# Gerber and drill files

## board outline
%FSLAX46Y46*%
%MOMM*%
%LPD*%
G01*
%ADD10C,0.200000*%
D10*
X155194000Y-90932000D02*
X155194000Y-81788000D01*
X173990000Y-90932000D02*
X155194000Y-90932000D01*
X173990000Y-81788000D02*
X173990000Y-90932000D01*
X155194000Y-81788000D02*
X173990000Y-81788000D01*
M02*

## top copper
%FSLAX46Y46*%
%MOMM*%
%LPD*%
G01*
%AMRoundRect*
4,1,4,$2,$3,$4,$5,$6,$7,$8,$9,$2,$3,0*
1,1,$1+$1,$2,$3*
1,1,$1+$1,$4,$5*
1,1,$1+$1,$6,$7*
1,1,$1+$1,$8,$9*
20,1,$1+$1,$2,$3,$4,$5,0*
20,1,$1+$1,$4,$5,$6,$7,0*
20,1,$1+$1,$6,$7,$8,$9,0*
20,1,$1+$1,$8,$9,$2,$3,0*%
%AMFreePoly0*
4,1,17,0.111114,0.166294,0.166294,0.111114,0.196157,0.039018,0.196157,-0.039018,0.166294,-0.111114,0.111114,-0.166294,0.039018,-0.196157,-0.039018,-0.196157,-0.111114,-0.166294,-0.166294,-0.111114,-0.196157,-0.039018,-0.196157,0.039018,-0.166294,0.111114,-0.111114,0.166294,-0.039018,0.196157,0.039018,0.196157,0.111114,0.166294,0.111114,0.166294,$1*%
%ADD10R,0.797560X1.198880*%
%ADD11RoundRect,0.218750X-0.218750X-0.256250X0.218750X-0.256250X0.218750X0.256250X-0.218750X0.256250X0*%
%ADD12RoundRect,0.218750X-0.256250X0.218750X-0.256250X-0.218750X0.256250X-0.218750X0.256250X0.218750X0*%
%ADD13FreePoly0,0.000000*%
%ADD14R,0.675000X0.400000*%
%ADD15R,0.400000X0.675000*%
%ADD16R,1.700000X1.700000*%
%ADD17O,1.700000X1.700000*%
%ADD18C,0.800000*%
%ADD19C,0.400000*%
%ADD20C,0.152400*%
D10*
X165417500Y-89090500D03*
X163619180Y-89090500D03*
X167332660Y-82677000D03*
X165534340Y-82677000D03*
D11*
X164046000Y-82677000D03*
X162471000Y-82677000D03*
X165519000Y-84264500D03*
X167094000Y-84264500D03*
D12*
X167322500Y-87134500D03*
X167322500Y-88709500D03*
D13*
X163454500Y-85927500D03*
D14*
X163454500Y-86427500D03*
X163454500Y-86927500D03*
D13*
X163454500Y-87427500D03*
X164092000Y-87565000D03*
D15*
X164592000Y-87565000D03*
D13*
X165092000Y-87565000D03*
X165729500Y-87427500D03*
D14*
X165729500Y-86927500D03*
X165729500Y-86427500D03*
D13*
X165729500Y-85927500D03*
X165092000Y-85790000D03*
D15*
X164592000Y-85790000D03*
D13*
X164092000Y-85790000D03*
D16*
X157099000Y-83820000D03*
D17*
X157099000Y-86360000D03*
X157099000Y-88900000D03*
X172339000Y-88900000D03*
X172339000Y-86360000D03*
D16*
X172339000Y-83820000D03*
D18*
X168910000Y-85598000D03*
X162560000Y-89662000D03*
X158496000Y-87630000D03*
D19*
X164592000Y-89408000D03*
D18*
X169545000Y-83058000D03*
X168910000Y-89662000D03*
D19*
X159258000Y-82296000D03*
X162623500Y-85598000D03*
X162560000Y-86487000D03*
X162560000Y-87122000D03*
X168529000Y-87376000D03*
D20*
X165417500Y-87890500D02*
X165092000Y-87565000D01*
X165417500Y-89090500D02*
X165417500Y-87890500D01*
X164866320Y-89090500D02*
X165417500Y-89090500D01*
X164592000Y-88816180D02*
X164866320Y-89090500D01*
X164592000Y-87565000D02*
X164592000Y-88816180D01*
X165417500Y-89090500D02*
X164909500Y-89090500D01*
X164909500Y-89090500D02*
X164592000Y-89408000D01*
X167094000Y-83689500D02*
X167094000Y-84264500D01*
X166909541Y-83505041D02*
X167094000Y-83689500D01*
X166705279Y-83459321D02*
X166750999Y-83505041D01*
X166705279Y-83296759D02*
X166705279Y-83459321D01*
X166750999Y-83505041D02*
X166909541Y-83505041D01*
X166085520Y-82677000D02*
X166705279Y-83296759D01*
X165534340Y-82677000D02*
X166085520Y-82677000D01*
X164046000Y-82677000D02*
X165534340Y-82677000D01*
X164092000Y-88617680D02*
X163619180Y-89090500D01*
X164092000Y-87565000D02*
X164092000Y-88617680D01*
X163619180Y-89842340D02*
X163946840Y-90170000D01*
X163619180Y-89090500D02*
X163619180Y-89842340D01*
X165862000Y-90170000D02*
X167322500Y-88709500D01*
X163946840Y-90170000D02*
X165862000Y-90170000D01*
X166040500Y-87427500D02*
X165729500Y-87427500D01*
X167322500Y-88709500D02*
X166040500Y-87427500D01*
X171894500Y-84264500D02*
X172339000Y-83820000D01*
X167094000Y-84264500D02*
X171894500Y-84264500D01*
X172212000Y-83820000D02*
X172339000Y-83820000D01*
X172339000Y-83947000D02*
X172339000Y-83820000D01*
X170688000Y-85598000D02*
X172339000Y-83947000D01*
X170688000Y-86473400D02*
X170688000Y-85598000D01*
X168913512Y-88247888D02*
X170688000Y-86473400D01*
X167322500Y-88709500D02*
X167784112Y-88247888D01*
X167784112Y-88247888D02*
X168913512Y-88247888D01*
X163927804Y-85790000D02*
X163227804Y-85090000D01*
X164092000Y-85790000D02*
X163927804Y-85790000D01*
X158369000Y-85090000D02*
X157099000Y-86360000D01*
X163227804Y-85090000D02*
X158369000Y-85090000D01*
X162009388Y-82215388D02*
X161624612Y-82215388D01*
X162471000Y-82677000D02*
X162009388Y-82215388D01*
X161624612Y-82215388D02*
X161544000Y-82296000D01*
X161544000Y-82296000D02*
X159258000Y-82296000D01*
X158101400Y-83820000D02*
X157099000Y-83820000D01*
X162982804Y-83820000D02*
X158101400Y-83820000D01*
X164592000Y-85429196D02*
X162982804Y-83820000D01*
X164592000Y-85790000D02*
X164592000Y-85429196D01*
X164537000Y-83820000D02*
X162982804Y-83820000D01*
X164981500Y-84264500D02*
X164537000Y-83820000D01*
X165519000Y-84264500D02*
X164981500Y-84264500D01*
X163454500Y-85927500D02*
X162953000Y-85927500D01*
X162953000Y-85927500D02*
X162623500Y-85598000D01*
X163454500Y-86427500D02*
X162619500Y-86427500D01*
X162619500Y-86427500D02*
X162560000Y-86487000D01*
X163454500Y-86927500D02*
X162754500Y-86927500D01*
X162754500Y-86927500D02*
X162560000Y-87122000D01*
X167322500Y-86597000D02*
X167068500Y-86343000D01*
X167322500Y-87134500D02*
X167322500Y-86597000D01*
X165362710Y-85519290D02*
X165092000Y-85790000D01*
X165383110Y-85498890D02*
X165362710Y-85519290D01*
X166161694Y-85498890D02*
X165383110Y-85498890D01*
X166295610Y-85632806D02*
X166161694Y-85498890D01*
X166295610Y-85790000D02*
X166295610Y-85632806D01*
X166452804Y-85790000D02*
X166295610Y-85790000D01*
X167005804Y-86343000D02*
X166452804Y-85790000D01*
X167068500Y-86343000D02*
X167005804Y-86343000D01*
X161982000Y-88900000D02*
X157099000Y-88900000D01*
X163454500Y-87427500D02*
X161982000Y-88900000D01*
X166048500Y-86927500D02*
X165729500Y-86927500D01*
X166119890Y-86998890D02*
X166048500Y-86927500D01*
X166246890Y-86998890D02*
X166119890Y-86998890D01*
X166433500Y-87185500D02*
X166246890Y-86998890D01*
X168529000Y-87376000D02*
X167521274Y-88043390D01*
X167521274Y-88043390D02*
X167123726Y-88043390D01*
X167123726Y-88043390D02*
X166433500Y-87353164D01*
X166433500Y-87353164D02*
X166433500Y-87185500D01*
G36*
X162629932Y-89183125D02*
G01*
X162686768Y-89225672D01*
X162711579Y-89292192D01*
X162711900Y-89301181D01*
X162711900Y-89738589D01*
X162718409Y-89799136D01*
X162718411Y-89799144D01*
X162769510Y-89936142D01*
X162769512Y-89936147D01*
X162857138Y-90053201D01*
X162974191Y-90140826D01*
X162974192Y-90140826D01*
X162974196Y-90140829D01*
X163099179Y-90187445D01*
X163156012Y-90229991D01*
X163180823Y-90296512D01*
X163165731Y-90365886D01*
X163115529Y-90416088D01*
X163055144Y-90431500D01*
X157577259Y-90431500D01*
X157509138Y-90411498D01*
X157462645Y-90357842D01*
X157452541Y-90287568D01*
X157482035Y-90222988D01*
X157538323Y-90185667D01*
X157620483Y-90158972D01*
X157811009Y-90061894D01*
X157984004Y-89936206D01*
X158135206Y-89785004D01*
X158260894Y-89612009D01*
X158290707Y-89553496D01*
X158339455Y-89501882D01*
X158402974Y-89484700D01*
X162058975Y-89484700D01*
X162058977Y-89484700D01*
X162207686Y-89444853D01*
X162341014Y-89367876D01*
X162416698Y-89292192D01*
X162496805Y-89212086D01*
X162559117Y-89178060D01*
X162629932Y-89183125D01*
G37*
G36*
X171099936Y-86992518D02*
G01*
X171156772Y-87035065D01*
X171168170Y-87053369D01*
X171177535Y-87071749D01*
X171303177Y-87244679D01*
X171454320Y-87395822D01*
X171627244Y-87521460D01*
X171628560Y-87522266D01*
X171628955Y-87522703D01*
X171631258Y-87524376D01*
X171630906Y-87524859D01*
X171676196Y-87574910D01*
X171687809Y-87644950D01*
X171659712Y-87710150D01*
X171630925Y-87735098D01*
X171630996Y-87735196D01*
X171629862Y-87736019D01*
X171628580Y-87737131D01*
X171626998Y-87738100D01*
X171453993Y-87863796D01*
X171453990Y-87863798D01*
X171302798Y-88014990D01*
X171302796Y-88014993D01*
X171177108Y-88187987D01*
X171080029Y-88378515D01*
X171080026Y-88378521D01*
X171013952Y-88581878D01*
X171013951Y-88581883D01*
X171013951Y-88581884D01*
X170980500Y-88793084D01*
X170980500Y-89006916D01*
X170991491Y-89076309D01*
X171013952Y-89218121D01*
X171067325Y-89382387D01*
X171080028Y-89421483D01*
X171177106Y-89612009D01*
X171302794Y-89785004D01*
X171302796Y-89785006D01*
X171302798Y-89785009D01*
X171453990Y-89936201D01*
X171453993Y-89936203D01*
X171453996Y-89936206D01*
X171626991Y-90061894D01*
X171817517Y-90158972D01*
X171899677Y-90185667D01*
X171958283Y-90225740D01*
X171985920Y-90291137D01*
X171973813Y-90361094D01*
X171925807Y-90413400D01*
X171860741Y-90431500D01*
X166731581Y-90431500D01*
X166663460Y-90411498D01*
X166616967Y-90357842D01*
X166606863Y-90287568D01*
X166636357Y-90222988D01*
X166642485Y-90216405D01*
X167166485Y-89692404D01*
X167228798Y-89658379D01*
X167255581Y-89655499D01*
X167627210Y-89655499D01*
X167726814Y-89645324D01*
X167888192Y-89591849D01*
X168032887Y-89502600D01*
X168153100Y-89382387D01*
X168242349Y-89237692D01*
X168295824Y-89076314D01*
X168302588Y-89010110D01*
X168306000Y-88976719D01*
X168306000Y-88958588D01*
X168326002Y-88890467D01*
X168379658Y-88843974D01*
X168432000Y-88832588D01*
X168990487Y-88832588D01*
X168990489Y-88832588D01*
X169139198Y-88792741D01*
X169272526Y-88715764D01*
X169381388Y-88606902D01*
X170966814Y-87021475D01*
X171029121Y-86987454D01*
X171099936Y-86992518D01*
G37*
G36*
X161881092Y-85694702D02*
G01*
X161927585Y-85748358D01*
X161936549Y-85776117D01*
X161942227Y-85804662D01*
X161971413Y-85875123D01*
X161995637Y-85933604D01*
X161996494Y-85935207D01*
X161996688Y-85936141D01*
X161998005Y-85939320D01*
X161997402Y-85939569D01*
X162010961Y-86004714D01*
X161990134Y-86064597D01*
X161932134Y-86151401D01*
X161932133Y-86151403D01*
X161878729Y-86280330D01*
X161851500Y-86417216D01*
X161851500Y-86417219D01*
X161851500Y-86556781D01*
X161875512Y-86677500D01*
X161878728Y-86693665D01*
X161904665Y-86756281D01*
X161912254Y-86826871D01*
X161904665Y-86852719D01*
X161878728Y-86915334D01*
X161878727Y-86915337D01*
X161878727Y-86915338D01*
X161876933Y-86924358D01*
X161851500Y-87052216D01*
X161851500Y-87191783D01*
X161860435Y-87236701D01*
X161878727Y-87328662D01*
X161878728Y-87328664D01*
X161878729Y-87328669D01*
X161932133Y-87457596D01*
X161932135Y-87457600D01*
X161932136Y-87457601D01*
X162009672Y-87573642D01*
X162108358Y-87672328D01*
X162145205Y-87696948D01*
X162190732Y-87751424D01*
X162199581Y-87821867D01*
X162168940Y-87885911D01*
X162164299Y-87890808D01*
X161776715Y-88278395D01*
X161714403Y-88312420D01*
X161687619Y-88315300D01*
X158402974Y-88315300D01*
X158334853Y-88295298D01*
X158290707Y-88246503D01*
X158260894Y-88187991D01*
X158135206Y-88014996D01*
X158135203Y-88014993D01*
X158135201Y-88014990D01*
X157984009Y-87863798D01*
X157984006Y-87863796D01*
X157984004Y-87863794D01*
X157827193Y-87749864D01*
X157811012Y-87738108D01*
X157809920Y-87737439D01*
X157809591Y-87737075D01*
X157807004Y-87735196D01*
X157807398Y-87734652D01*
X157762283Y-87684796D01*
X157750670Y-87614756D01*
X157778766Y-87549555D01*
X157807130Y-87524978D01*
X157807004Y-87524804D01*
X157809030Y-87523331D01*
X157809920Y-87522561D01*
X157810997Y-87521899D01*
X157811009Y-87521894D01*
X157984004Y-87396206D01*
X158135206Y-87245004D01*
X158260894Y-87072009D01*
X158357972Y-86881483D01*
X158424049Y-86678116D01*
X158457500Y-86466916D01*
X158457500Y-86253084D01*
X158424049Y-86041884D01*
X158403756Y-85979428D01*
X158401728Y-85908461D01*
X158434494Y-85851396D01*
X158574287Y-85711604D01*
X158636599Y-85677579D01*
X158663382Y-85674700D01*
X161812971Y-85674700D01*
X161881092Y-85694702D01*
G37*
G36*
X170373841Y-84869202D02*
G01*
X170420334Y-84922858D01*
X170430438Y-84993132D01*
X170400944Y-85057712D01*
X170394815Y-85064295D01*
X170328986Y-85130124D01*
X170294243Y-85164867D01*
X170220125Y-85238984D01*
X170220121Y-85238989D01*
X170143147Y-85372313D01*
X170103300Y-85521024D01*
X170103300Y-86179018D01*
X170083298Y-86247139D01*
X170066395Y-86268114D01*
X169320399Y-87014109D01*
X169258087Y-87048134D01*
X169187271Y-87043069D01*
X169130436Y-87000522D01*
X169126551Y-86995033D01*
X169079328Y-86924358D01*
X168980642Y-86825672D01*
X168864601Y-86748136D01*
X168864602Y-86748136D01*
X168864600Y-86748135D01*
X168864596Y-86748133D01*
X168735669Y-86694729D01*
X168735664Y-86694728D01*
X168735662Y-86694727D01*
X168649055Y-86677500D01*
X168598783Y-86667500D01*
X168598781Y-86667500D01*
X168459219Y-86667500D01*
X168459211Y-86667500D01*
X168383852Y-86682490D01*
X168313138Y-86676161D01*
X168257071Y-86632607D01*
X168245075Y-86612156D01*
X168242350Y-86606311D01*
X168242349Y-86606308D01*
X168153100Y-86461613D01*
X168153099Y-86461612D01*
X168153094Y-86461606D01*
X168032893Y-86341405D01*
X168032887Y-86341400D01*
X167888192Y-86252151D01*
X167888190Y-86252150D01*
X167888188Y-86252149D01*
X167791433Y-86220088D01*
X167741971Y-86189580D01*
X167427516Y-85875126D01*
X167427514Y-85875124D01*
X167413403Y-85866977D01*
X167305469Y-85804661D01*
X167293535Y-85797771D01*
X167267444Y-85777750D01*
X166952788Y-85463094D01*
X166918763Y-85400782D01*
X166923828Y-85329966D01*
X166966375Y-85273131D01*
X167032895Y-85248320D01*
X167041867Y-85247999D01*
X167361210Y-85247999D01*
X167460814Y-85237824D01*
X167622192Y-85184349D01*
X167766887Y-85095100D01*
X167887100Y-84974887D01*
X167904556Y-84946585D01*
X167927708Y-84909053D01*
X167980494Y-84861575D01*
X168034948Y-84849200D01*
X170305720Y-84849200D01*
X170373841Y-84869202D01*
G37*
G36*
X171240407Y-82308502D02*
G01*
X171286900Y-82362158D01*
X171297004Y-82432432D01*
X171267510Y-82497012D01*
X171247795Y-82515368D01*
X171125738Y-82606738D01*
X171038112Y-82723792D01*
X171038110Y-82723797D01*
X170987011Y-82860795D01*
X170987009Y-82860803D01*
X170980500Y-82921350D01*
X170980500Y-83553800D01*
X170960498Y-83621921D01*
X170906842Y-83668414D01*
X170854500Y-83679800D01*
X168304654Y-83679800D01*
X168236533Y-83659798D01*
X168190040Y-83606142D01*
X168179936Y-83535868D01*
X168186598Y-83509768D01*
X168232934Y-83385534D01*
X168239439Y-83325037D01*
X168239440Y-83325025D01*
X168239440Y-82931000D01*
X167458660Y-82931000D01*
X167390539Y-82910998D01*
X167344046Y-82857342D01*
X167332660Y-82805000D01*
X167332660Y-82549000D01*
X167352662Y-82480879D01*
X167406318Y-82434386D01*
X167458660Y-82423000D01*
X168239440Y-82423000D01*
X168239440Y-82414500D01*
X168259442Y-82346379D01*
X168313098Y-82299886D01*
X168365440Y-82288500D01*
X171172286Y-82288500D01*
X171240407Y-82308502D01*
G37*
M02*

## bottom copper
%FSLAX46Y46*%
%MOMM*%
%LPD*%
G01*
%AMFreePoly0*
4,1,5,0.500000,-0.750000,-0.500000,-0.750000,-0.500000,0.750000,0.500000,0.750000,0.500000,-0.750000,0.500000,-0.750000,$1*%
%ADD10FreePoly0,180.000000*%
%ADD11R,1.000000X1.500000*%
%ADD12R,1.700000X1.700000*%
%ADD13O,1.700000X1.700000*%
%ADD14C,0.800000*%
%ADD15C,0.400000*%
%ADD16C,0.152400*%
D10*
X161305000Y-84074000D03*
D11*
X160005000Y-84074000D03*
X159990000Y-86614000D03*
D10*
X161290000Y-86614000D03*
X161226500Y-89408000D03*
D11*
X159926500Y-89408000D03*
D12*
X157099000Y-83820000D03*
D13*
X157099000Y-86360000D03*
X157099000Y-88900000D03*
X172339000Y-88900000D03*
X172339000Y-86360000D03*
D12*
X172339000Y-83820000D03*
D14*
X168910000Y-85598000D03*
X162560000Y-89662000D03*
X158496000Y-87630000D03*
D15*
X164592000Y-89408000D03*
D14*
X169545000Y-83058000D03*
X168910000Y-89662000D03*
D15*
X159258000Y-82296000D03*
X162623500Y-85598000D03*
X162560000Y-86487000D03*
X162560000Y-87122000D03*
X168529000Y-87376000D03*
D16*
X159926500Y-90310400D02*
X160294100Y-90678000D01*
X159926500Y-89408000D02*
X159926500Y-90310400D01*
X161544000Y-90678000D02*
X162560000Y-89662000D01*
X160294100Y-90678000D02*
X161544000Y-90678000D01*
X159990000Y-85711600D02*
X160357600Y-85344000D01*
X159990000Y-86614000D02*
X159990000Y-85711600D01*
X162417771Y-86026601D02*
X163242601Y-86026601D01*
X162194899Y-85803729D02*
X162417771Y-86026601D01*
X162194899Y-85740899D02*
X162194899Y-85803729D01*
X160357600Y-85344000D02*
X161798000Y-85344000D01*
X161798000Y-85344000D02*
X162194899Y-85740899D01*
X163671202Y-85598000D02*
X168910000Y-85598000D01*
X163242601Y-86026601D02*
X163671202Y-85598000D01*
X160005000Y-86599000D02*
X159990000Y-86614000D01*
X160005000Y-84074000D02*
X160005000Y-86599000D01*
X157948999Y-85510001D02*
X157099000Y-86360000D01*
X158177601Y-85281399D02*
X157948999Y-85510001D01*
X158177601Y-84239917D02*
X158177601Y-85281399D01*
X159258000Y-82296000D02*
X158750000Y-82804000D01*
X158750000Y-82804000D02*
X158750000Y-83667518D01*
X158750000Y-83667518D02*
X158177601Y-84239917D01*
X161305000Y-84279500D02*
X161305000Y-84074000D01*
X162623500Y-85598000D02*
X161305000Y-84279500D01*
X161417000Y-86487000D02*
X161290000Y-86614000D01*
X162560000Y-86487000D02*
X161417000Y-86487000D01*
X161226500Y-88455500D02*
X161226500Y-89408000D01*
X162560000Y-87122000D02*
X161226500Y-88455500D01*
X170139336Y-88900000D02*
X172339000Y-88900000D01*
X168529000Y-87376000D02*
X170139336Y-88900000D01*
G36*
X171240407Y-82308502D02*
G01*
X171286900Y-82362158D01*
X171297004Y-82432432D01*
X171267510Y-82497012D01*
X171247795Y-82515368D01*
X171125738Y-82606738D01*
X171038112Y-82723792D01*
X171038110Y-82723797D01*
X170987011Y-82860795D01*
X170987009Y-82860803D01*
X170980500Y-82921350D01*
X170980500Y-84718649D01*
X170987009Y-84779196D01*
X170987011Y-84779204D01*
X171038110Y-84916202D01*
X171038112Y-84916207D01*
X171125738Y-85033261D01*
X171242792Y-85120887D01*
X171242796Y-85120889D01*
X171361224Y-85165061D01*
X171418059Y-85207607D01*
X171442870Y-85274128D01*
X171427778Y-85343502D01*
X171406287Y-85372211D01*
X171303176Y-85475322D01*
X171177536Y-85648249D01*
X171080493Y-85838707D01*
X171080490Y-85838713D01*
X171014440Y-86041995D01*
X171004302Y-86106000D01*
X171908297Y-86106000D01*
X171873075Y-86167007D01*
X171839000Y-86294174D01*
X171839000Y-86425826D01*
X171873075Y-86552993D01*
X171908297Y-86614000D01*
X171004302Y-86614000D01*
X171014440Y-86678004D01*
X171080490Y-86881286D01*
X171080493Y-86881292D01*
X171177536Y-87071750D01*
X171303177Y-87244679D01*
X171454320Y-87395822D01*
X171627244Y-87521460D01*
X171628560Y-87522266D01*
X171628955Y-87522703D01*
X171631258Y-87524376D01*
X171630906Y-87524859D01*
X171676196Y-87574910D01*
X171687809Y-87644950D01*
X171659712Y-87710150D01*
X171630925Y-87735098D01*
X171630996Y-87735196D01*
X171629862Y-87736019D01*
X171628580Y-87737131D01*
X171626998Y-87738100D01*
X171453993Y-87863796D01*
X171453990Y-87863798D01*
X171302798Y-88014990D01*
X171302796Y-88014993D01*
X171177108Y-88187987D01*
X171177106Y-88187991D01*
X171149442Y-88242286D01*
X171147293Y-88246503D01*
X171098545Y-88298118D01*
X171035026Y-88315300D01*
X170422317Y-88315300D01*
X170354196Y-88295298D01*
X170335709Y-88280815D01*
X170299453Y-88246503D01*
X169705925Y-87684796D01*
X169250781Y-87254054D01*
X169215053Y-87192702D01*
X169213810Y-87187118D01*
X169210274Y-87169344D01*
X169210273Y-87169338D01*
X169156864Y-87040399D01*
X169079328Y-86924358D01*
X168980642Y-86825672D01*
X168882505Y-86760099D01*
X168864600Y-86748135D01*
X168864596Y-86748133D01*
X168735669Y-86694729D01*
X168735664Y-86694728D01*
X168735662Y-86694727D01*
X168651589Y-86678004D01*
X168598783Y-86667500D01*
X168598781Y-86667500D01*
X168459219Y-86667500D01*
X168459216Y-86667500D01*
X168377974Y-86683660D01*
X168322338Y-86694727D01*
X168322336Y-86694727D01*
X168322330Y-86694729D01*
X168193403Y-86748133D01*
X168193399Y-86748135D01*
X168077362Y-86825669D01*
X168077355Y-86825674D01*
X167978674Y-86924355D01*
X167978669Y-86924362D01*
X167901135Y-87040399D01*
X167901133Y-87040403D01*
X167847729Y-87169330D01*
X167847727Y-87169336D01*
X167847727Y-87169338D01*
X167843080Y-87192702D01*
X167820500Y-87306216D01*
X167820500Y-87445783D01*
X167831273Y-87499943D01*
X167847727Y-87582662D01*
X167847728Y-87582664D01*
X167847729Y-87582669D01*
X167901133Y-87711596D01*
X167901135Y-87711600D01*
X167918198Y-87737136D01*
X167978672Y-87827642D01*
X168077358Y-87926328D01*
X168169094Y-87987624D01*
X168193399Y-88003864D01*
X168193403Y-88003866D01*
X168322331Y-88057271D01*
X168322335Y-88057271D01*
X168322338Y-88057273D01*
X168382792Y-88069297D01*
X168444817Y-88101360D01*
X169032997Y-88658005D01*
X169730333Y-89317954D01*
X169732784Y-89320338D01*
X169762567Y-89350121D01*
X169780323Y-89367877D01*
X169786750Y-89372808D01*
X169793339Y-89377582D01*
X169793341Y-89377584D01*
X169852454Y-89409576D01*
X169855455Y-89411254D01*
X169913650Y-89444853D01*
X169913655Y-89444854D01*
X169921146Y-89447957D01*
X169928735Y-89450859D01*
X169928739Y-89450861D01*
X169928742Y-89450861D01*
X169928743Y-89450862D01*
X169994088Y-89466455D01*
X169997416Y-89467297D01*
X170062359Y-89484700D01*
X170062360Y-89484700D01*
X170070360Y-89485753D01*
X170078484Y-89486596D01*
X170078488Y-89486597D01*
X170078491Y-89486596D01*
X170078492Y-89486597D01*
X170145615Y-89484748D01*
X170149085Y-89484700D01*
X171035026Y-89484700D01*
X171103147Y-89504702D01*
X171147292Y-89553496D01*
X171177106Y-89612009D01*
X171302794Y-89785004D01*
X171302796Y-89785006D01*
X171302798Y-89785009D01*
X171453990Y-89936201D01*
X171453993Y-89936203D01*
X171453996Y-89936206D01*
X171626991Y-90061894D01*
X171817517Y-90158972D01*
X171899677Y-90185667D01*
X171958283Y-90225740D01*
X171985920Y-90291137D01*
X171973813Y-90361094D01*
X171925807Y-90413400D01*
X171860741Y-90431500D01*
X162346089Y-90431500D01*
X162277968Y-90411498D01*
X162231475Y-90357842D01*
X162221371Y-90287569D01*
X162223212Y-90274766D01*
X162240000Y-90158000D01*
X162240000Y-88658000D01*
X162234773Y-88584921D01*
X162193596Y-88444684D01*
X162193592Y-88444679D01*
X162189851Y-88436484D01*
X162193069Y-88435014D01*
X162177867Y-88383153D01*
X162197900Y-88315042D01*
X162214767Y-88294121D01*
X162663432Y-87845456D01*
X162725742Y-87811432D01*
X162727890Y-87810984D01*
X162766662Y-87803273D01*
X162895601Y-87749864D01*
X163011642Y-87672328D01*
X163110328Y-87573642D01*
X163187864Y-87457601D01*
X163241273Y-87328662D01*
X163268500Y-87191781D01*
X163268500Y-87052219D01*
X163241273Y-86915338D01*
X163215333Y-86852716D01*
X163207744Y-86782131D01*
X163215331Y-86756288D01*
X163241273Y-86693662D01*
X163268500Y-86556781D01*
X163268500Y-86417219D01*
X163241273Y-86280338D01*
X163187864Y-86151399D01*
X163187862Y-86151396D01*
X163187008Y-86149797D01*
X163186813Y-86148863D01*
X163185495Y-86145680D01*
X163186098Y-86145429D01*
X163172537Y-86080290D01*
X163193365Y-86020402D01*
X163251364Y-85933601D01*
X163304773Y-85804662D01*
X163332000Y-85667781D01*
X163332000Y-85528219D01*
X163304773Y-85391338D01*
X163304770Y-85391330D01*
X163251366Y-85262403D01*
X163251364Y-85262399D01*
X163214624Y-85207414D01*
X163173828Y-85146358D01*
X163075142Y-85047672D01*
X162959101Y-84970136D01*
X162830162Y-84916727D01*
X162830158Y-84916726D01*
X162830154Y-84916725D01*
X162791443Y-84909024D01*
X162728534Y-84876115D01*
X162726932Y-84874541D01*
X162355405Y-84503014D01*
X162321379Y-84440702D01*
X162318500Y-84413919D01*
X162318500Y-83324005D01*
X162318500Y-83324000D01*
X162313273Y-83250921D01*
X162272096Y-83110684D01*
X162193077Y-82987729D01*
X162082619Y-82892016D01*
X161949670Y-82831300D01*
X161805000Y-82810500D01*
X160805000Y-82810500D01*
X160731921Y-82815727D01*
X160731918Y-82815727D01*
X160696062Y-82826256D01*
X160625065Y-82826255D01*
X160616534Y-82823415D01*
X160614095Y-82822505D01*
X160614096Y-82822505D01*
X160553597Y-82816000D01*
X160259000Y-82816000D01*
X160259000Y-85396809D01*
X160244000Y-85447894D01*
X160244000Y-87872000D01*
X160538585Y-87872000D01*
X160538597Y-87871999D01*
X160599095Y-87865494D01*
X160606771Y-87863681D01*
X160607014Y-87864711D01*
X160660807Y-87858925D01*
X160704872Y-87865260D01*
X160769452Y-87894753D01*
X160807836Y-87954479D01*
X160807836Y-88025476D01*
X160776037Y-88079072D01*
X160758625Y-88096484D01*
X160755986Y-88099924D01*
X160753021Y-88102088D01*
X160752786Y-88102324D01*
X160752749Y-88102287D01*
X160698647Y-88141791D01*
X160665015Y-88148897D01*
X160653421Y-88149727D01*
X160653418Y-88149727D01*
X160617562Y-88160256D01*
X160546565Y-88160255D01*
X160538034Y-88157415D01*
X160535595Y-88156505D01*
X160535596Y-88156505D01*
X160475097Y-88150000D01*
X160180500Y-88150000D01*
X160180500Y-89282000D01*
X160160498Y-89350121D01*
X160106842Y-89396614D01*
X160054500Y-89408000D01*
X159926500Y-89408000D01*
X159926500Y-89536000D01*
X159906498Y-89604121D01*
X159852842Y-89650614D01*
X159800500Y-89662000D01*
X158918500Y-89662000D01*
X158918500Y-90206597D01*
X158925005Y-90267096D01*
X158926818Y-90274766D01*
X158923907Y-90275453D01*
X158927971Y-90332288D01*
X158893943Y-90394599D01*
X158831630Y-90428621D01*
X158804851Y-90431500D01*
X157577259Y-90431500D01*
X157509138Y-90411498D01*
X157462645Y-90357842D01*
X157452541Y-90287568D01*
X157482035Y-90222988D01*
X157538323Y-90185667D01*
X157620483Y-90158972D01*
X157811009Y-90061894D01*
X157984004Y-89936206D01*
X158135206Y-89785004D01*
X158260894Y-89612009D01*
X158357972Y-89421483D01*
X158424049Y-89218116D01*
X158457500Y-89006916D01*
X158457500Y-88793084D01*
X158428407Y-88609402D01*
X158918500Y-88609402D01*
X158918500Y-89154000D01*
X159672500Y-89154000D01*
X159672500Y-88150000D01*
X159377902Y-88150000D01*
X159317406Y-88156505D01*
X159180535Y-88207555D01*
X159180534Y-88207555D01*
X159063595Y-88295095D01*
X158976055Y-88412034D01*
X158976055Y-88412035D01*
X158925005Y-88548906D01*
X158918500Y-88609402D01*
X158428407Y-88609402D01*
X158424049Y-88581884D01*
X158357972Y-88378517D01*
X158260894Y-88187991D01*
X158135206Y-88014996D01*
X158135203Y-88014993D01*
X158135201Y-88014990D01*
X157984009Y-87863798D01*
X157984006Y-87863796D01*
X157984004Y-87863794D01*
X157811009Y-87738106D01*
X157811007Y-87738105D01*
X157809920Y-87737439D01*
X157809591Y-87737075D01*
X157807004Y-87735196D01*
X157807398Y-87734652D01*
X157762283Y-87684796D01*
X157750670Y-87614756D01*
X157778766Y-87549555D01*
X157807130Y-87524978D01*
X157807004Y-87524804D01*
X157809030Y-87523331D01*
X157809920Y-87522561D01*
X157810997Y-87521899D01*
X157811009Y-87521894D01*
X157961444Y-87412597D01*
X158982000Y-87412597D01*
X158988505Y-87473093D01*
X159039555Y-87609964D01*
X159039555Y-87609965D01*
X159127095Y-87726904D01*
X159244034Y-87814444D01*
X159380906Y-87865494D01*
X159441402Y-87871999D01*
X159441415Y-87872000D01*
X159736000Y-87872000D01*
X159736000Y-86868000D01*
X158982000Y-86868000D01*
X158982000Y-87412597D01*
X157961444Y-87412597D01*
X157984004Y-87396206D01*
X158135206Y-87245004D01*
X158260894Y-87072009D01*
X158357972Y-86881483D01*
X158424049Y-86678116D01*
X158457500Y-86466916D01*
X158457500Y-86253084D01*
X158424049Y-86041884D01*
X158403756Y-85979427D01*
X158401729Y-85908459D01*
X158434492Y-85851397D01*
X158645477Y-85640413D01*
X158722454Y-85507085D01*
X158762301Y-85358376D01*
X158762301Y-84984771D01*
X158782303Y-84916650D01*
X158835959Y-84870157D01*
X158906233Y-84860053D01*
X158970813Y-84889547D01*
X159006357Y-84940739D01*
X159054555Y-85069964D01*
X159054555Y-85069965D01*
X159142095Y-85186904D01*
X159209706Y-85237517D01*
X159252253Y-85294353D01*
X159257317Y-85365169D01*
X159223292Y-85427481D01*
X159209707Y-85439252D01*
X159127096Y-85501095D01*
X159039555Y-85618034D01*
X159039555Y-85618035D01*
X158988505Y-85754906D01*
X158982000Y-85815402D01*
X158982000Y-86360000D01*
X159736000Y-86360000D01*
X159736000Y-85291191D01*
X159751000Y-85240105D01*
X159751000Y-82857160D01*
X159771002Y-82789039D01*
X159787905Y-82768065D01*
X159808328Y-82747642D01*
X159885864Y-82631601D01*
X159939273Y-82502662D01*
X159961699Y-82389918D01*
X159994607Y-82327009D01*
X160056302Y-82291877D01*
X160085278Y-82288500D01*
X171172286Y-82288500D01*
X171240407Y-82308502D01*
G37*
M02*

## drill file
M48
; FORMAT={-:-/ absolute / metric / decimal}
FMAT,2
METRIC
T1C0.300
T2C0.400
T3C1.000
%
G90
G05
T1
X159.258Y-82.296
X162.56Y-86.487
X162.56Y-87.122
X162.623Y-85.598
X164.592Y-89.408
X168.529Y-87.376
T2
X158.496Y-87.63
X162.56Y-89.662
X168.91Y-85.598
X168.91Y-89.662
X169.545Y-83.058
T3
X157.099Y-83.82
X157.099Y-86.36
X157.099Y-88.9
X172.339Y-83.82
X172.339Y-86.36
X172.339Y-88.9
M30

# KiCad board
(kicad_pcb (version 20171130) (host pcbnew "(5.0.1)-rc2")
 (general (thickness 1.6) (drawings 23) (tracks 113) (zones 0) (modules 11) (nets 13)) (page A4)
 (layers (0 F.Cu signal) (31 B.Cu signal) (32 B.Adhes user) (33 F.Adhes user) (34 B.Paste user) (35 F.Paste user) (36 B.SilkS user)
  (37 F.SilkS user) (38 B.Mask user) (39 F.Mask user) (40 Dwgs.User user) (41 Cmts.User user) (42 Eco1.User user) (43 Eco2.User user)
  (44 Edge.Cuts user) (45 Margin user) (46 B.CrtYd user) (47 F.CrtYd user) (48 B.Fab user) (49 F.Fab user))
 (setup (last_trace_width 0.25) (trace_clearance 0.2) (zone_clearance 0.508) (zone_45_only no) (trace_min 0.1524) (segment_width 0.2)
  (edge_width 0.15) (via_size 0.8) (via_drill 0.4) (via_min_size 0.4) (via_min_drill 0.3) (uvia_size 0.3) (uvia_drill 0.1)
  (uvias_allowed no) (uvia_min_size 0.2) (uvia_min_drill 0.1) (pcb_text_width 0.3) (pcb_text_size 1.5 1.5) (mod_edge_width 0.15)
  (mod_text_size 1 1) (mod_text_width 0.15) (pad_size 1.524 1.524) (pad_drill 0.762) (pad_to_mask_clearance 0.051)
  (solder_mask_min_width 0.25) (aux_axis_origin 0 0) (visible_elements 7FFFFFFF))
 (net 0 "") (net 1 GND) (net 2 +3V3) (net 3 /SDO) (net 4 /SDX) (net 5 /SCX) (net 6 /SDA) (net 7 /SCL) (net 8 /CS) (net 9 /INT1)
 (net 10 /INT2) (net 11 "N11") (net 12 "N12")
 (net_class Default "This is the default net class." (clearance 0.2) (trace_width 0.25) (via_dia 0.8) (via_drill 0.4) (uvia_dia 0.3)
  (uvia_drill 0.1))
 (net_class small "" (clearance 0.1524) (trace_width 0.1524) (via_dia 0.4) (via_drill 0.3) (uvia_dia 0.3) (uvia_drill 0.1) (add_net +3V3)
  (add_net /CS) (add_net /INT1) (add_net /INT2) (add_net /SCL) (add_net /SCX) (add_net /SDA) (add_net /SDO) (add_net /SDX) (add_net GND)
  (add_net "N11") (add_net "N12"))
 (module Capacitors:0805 (layer F.Cu) (at 164.51834 89.0905 180)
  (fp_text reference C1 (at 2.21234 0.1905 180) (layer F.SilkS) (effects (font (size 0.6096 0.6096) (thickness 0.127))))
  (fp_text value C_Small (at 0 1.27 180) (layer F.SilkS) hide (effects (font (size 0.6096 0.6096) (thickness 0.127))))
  (pad 1 smd rect (at -0.89916 0 180) (size 0.79756 1.19888) (layers F.Cu F.Paste F.Mask) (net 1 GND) (solder_mask_margin 0.1016))
  (pad 2 smd rect (at 0.89916 0 180) (size 0.79756 1.19888) (layers F.Cu F.Paste F.Mask) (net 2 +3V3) (solder_mask_margin 0.1016)))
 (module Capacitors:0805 (layer F.Cu) (at 166.4335 82.677)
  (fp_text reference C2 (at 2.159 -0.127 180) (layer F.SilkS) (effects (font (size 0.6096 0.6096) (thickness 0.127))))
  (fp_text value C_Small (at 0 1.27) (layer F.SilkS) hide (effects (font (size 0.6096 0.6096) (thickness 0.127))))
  (pad 2 smd rect (at 0.89916 0) (size 0.79756 1.19888) (layers F.Cu F.Paste F.Mask) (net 1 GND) (solder_mask_margin 0.1016))
  (pad 1 smd rect (at -0.89916 0) (size 0.79756 1.19888) (layers F.Cu F.Paste F.Mask) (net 2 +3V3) (solder_mask_margin 0.1016)))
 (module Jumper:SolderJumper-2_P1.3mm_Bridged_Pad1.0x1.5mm (layer B.Cu) (at 160.655 84.074 180)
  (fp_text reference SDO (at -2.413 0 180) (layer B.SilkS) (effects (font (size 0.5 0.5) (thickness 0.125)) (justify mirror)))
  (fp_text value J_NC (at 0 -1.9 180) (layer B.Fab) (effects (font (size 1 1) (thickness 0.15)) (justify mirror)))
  (pad 1 smd custom (at -0.65 0 180) (size 1 1.5) (layers B.Cu B.Mask) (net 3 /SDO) (options (clearance outline) (anchor rect)) (primitives))
  (pad 2 smd rect (at 0.65 0 180) (size 1 1.5) (layers B.Cu B.Mask) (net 1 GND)))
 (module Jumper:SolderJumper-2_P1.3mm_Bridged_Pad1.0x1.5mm (layer B.Cu) (at 160.64 86.614 180)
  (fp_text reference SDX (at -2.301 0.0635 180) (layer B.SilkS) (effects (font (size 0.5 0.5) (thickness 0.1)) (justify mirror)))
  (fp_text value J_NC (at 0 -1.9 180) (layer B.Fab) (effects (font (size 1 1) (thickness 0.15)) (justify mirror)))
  (pad 2 smd rect (at 0.65 0 180) (size 1 1.5) (layers B.Cu B.Mask) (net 1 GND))
  (pad 1 smd custom (at -0.65 0 180) (size 1 1.5) (layers B.Cu B.Mask) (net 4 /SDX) (options (clearance outline) (anchor rect)) (primitives)))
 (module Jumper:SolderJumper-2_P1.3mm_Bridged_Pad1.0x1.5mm (layer B.Cu) (at 160.5765 89.408 180)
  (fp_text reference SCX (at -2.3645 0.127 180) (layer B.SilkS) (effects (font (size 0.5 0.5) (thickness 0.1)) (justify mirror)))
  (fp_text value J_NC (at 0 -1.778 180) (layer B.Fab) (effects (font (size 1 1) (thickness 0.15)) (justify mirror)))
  (pad 1 smd custom (at -0.65 0 180) (size 1 1.5) (layers B.Cu B.Mask) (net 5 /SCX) (options (clearance outline) (anchor rect)) (primitives))
  (pad 2 smd rect (at 0.65 0 180) (size 1 1.5) (layers B.Cu B.Mask) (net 1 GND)))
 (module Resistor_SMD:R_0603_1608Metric (layer F.Cu) (at 163.2585 82.677)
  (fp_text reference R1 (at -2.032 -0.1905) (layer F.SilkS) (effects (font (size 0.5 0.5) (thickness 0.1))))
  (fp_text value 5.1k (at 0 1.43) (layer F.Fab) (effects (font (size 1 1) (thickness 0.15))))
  (pad 2 smd roundrect (at 0.7875 0) (size 0.875 0.95) (layers F.Cu F.Paste F.Mask) (roundrect_rratio 0.25) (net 2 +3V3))
  (pad 1 smd roundrect (at -0.7875 0) (size 0.875 0.95) (layers F.Cu F.Paste F.Mask) (roundrect_rratio 0.25) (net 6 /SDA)))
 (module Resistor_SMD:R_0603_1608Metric (layer F.Cu) (at 166.3065 84.2645)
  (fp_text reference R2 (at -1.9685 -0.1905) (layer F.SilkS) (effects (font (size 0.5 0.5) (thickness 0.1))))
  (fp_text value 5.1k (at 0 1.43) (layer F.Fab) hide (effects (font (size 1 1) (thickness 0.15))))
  (pad 1 smd roundrect (at -0.7875 0) (size 0.875 0.95) (layers F.Cu F.Paste F.Mask) (roundrect_rratio 0.25) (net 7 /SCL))
  (pad 2 smd roundrect (at 0.7875 0) (size 0.875 0.95) (layers F.Cu F.Paste F.Mask) (roundrect_rratio 0.25) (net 2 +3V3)))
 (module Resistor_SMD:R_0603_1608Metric (layer F.Cu) (at 167.3225 87.922 270)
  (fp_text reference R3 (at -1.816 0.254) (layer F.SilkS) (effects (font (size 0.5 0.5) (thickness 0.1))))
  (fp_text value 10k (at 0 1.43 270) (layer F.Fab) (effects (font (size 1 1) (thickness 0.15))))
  (pad 1 smd roundrect (at -0.7875 0 270) (size 0.875 0.95) (layers F.Cu F.Paste F.Mask) (roundrect_rratio 0.25) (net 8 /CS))
  (pad 2 smd roundrect (at 0.7875 0 270) (size 0.875 0.95) (layers F.Cu F.Paste F.Mask) (roundrect_rratio 0.25) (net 2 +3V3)))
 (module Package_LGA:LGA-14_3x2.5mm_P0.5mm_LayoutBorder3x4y (layer F.Cu) (at 164.592 86.6775)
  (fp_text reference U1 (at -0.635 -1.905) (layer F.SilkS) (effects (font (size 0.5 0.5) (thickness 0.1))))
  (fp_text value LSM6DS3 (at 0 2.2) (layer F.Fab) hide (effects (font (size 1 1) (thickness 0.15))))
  (pad 1 smd custom (at -1.1375 -0.75) (size 0.4 0.4) (layers F.Cu F.Paste F.Mask) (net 3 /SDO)
   (options (clearance outline) (anchor circle)) (primitives))
  (pad 2 smd rect (at -1.1375 -0.25) (size 0.675 0.4) (layers F.Cu F.Paste F.Mask) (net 4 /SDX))
  (pad 3 smd rect (at -1.1375 0.25) (size 0.675 0.4) (layers F.Cu F.Paste F.Mask) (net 5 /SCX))
  (pad 4 smd custom (at -1.1375 0.75) (size 0.4 0.4) (layers F.Cu F.Paste F.Mask) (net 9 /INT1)
   (options (clearance outline) (anchor circle)) (primitives))
  (pad 5 smd custom (at -0.5 0.8875) (size 0.4 0.4) (layers F.Cu F.Paste F.Mask) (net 2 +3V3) (options (clearance outline) (anchor circle))
   (primitives))
  (pad 6 smd rect (at 0 0.8875) (size 0.4 0.675) (layers F.Cu F.Paste F.Mask) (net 1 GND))
  (pad 7 smd custom (at 0.5 0.8875) (size 0.4 0.4) (layers F.Cu F.Paste F.Mask) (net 1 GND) (options (clearance outline) (anchor circle))
   (primitives))
  (pad 8 smd custom (at 1.1375 0.75) (size 0.4 0.4) (layers F.Cu F.Paste F.Mask) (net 2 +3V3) (options (clearance outline) (anchor circle))
   (primitives))
  (pad 9 smd rect (at 1.1375 0.25) (size 0.675 0.4) (layers F.Cu F.Paste F.Mask) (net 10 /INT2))
  (pad 10 smd rect (at 1.1375 -0.25) (size 0.675 0.4) (layers F.Cu F.Paste F.Mask) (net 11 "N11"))
  (pad 11 smd custom (at 1.1375 -0.75) (size 0.4 0.4) (layers F.Cu F.Paste F.Mask) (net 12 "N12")
   (options (clearance outline) (anchor circle)) (primitives))
  (pad 12 smd custom (at 0.5 -0.8875) (size 0.4 0.4) (layers F.Cu F.Paste F.Mask) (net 8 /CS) (options (clearance outline) (anchor circle))
   (primitives))
  (pad 13 smd rect (at 0 -0.8875) (size 0.4 0.675) (layers F.Cu F.Paste F.Mask) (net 7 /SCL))
  (pad 14 smd custom (at -0.5 -0.8875) (size 0.4 0.4) (layers F.Cu F.Paste F.Mask) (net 6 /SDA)
   (options (clearance outline) (anchor circle)) (primitives)))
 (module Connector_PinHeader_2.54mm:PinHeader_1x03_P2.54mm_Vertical (layer F.Cu) (at 157.099 83.82)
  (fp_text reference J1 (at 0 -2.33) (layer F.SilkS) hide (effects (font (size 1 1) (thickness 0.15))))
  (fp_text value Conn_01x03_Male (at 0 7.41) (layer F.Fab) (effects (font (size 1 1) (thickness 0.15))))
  (pad 1 thru_hole rect (at 0 0) (size 1.7 1.7) (drill 1) (layers *.Cu *.Mask) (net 7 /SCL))
  (pad 2 thru_hole oval (at 0 2.54) (size 1.7 1.7) (drill 1) (layers *.Cu *.Mask) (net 6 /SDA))
  (pad 3 thru_hole oval (at 0 5.08) (size 1.7 1.7) (drill 1) (layers *.Cu *.Mask) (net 9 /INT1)))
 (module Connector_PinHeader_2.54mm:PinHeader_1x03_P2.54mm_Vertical (layer F.Cu) (at 172.339 83.82)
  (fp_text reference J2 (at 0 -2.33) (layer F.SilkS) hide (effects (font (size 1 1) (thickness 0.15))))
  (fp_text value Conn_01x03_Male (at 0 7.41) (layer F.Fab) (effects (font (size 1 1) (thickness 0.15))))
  (pad 3 thru_hole oval (at 0 5.08) (size 1.7 1.7) (drill 1) (layers *.Cu *.Mask) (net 10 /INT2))
  (pad 2 thru_hole oval (at 0 2.54) (size 1.7 1.7) (drill 1) (layers *.Cu *.Mask) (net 1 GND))
  (pad 1 thru_hole rect (at 0 0) (size 1.7 1.7) (drill 1) (layers *.Cu *.Mask) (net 2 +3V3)))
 (gr_line (start 155.194 90.932) (end 155.194 81.788) (layer Edge.Cuts) (width 0.2))
 (gr_line (start 173.99 90.932) (end 155.194 90.932) (layer Edge.Cuts) (width 0.2))
 (gr_line (start 173.99 81.788) (end 173.99 90.932) (layer Edge.Cuts) (width 0.2))
 (gr_line (start 155.194 81.788) (end 173.99 81.788) (layer Edge.Cuts) (width 0.2))
 (via (at 168.91 85.598) (size 0.8) (drill 0.4) (layers F.Cu B.Cu) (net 1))
 (segment (start 165.4175 87.8905) (end 165.092 87.565) (width 0.1524) (layer F.Cu) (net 1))
 (segment (start 165.4175 89.0905) (end 165.4175 87.8905) (width 0.1524) (layer F.Cu) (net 1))
 (segment (start 164.86632 89.0905) (end 165.4175 89.0905) (width 0.1524) (layer F.Cu) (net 1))
 (segment (start 164.592 88.81618) (end 164.86632 89.0905) (width 0.1524) (layer F.Cu) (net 1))
 (segment (start 164.592 87.565) (end 164.592 88.81618) (width 0.1524) (layer F.Cu) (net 1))
 (via (at 162.56 89.662) (size 0.8) (drill 0.4) (layers F.Cu B.Cu) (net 1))
 (via (at 158.496 87.63) (size 0.8) (drill 0.4) (layers F.Cu B.Cu) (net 1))
 (segment (start 159.9265 90.3104) (end 160.2941 90.678) (width 0.1524) (layer B.Cu) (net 1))
 (segment (start 159.9265 89.408) (end 159.9265 90.3104) (width 0.1524) (layer B.Cu) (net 1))
 (segment (start 161.544 90.678) (end 162.56 89.662) (width 0.1524) (layer B.Cu) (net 1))
 (segment (start 160.2941 90.678) (end 161.544 90.678) (width 0.1524) (layer B.Cu) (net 1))
 (segment (start 159.99 85.7116) (end 160.3576 85.344) (width 0.1524) (layer B.Cu) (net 1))
 (segment (start 159.99 86.614) (end 159.99 85.7116) (width 0.1524) (layer B.Cu) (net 1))
 (segment (start 162.417771 86.026601) (end 163.242601 86.026601) (width 0.1524) (layer B.Cu) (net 1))
 (segment (start 162.194899 85.803729) (end 162.417771 86.026601) (width 0.1524) (layer B.Cu) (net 1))
 (segment (start 162.194899 85.740899) (end 162.194899 85.803729) (width 0.1524) (layer B.Cu) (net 1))
 (segment (start 160.3576 85.344) (end 161.798 85.344) (width 0.1524) (layer B.Cu) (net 1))
 (segment (start 161.798 85.344) (end 162.194899 85.740899) (width 0.1524) (layer B.Cu) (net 1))
 (segment (start 163.671202 85.598) (end 168.91 85.598) (width 0.1524) (layer B.Cu) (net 1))
 (segment (start 163.242601 86.026601) (end 163.671202 85.598) (width 0.1524) (layer B.Cu) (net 1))
 (segment (start 160.005 86.599) (end 159.99 86.614) (width 0.1524) (layer B.Cu) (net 1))
 (segment (start 160.005 84.074) (end 160.005 86.599) (width 0.1524) (layer B.Cu) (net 1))
 (via (at 164.592 89.408) (size 0.4) (drill 0.3) (layers F.Cu B.Cu) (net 1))
 (segment (start 165.4175 89.0905) (end 164.9095 89.0905) (width 0.1524) (layer F.Cu) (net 1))
 (segment (start 164.9095 89.0905) (end 164.592 89.408) (width 0.1524) (layer F.Cu) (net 1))
 (via (at 169.545 83.058) (size 0.8) (drill 0.4) (layers F.Cu B.Cu) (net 1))
 (via (at 168.91 89.662) (size 0.8) (drill 0.4) (layers F.Cu B.Cu) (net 1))
 (segment (start 167.094 83.6895) (end 167.094 84.2645) (width 0.1524) (layer F.Cu) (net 2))
 (segment (start 166.909541 83.505041) (end 167.094 83.6895) (width 0.1524) (layer F.Cu) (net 2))
 (segment (start 166.705279 83.459321) (end 166.750999 83.505041) (width 0.1524) (layer F.Cu) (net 2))
 (segment (start 166.705279 83.296759) (end 166.705279 83.459321) (width 0.1524) (layer F.Cu) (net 2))
 (segment (start 166.750999 83.505041) (end 166.909541 83.505041) (width 0.1524) (layer F.Cu) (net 2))
 (segment (start 166.08552 82.677) (end 166.705279 83.296759) (width 0.1524) (layer F.Cu) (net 2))
 (segment (start 165.53434 82.677) (end 166.08552 82.677) (width 0.1524) (layer F.Cu) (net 2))
 (segment (start 164.046 82.677) (end 165.53434 82.677) (width 0.1524) (layer F.Cu) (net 2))
 (segment (start 164.092 88.61768) (end 163.61918 89.0905) (width 0.1524) (layer F.Cu) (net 2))
 (segment (start 164.092 87.565) (end 164.092 88.61768) (width 0.1524) (layer F.Cu) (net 2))
 (segment (start 163.61918 89.84234) (end 163.94684 90.17) (width 0.1524) (layer F.Cu) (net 2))
 (segment (start 163.61918 89.0905) (end 163.61918 89.84234) (width 0.1524) (layer F.Cu) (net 2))
 (segment (start 165.862 90.17) (end 167.3225 88.7095) (width 0.1524) (layer F.Cu) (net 2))
 (segment (start 163.94684 90.17) (end 165.862 90.17) (width 0.1524) (layer F.Cu) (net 2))
 (segment (start 166.0405 87.4275) (end 165.7295 87.4275) (width 0.1524) (layer F.Cu) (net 2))
 (segment (start 167.3225 88.7095) (end 166.0405 87.4275) (width 0.1524) (layer F.Cu) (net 2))
 (segment (start 171.8945 84.2645) (end 172.339 83.82) (width 0.1524) (layer F.Cu) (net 2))
 (segment (start 167.094 84.2645) (end 171.8945 84.2645) (width 0.1524) (layer F.Cu) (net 2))
 (segment (start 172.212 83.82) (end 172.339 83.82) (width 0.1524) (layer F.Cu) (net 2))
 (segment (start 172.339 83.947) (end 172.339 83.82) (width 0.1524) (layer F.Cu) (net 2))
 (segment (start 170.688 85.598) (end 172.339 83.947) (width 0.1524) (layer F.Cu) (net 2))
 (segment (start 170.688 86.4734) (end 170.688 85.598) (width 0.1524) (layer F.Cu) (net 2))
 (segment (start 168.913512 88.247888) (end 170.688 86.4734) (width 0.1524) (layer F.Cu) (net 2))
 (segment (start 167.3225 88.7095) (end 167.784112 88.247888) (width 0.1524) (layer F.Cu) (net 2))
 (segment (start 167.784112 88.247888) (end 168.913512 88.247888) (width 0.1524) (layer F.Cu) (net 2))
 (segment (start 163.927804 85.79) (end 163.227804 85.09) (width 0.1524) (layer F.Cu) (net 6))
 (segment (start 164.092 85.79) (end 163.927804 85.79) (width 0.1524) (layer F.Cu) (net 6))
 (segment (start 158.369 85.09) (end 157.099 86.36) (width 0.1524) (layer F.Cu) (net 6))
 (segment (start 163.227804 85.09) (end 158.369 85.09) (width 0.1524) (layer F.Cu) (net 6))
 (segment (start 157.948999 85.510001) (end 157.099 86.36) (width 0.1524) (layer B.Cu) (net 6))
 (segment (start 158.177601 85.281399) (end 157.948999 85.510001) (width 0.1524) (layer B.Cu) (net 6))
 (segment (start 158.177601 84.239917) (end 158.177601 85.281399) (width 0.1524) (layer B.Cu) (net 6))
 (segment (start 162.009388 82.215388) (end 161.624612 82.215388) (width 0.1524) (layer F.Cu) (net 6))
 (segment (start 162.471 82.677) (end 162.009388 82.215388) (width 0.1524) (layer F.Cu) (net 6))
 (segment (start 161.624612 82.215388) (end 161.544 82.296) (width 0.1524) (layer F.Cu) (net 6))
 (via (at 159.258 82.296) (size 0.4) (drill 0.3) (layers F.Cu B.Cu) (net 6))
 (segment (start 161.544 82.296) (end 159.258 82.296) (width 0.1524) (layer F.Cu) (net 6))
 (segment (start 159.258 82.296) (end 158.75 82.804) (width 0.1524) (layer B.Cu) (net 6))
 (segment (start 158.75 82.804) (end 158.75 83.667518) (width 0.1524) (layer B.Cu) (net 6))
 (segment (start 158.75 83.667518) (end 158.177601 84.239917) (width 0.1524) (layer B.Cu) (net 6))
 (segment (start 158.1014 83.82) (end 157.099 83.82) (width 0.1524) (layer F.Cu) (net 7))
 (segment (start 162.982804 83.82) (end 158.1014 83.82) (width 0.1524) (layer F.Cu) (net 7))
 (segment (start 164.592 85.429196) (end 162.982804 83.82) (width 0.1524) (layer F.Cu) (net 7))
 (segment (start 164.592 85.79) (end 164.592 85.429196) (width 0.1524) (layer F.Cu) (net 7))
 (segment (start 164.537 83.82) (end 162.982804 83.82) (width 0.1524) (layer F.Cu) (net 7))
 (segment (start 164.9815 84.2645) (end 164.537 83.82) (width 0.1524) (layer F.Cu) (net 7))
 (segment (start 165.519 84.2645) (end 164.9815 84.2645) (width 0.1524) (layer F.Cu) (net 7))
 (via (at 162.6235 85.598) (size 0.4) (drill 0.3) (layers F.Cu B.Cu) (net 3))
 (segment (start 163.4545 85.9275) (end 162.953 85.9275) (width 0.1524) (layer F.Cu) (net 3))
 (segment (start 162.953 85.9275) (end 162.6235 85.598) (width 0.1524) (layer F.Cu) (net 3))
 (segment (start 161.305 84.2795) (end 161.305 84.074) (width 0.1524) (layer B.Cu) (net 3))
 (segment (start 162.6235 85.598) (end 161.305 84.2795) (width 0.1524) (layer B.Cu) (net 3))
 (via (at 162.56 86.487) (size 0.4) (drill 0.3) (layers F.Cu B.Cu) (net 4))
 (segment (start 163.4545 86.4275) (end 162.6195 86.4275) (width 0.1524) (layer F.Cu) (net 4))
 (segment (start 162.6195 86.4275) (end 162.56 86.487) (width 0.1524) (layer F.Cu) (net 4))
 (segment (start 161.417 86.487) (end 161.29 86.614) (width 0.1524) (layer B.Cu) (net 4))
 (segment (start 162.56 86.487) (end 161.417 86.487) (width 0.1524) (layer B.Cu) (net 4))
 (via (at 162.56 87.122) (size 0.4) (drill 0.3) (layers F.Cu B.Cu) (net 5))
 (segment (start 163.4545 86.9275) (end 162.7545 86.9275) (width 0.1524) (layer F.Cu) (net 5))
 (segment (start 162.7545 86.9275) (end 162.56 87.122) (width 0.1524) (layer F.Cu) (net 5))
 (segment (start 161.2265 88.4555) (end 161.2265 89.408) (width 0.1524) (layer B.Cu) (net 5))
 (segment (start 162.56 87.122) (end 161.2265 88.4555) (width 0.1524) (layer B.Cu) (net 5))
 (segment (start 167.3225 86.597) (end 167.0685 86.343) (width 0.1524) (layer F.Cu) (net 8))
 (segment (start 167.3225 87.1345) (end 167.3225 86.597) (width 0.1524) (layer F.Cu) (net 8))
 (segment (start 165.36271 85.51929) (end 165.092 85.79) (width 0.1524) (layer F.Cu) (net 8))
 (segment (start 165.38311 85.49889) (end 165.36271 85.51929) (width 0.1524) (layer F.Cu) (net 8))
 (segment (start 166.161694 85.49889) (end 165.38311 85.49889) (width 0.1524) (layer F.Cu) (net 8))
 (segment (start 166.29561 85.632806) (end 166.161694 85.49889) (width 0.1524) (layer F.Cu) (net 8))
 (segment (start 166.29561 85.79) (end 166.29561 85.632806) (width 0.1524) (layer F.Cu) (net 8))
 (segment (start 166.452804 85.79) (end 166.29561 85.79) (width 0.1524) (layer F.Cu) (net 8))
 (segment (start 167.005804 86.343) (end 166.452804 85.79) (width 0.1524) (layer F.Cu) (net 8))
 (segment (start 167.0685 86.343) (end 167.005804 86.343) (width 0.1524) (layer F.Cu) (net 8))
 (segment (start 161.982 88.9) (end 157.099 88.9) (width 0.1524) (layer F.Cu) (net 9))
 (segment (start 163.4545 87.4275) (end 161.982 88.9) (width 0.1524) (layer F.Cu) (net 9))
 (segment (start 170.139336 88.9) (end 172.339 88.9) (width 0.1524) (layer B.Cu) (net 10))
 (segment (start 168.529 87.376) (end 170.139336 88.9) (width 0.1524) (layer B.Cu) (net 10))
 (segment (start 166.0485 86.9275) (end 165.7295 86.9275) (width 0.1524) (layer F.Cu) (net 10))
 (segment (start 166.11989 86.99889) (end 166.0485 86.9275) (width 0.1524) (layer F.Cu) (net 10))
 (segment (start 166.24689 86.99889) (end 166.11989 86.99889) (width 0.1524) (layer F.Cu) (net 10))
 (segment (start 166.4335 87.1855) (end 166.24689 86.99889) (width 0.1524) (layer F.Cu) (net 10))
 (segment (start 168.529 87.376) (end 167.521274 88.04339) (width 0.1524) (layer F.Cu) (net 10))
 (segment (start 167.521274 88.04339) (end 167.123726 88.04339) (width 0.1524) (layer F.Cu) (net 10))
 (segment (start 167.123726 88.04339) (end 166.4335 87.353164) (width 0.1524) (layer F.Cu) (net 10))
 (segment (start 166.4335 87.353164) (end 166.4335 87.1855) (width 0.1524) (layer F.Cu) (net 10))
 (via (at 168.529 87.376) (size 0.4) (drill 0.3) (layers F.Cu B.Cu) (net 10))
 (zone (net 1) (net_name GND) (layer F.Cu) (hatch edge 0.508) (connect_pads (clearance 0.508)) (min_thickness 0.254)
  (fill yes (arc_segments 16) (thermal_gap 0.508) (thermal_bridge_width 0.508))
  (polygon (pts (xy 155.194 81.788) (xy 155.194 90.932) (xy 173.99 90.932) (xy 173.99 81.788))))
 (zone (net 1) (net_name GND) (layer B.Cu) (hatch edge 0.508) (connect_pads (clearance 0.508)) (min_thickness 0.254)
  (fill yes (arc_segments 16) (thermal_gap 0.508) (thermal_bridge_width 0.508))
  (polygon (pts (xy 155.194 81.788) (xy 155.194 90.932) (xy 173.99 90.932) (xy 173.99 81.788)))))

